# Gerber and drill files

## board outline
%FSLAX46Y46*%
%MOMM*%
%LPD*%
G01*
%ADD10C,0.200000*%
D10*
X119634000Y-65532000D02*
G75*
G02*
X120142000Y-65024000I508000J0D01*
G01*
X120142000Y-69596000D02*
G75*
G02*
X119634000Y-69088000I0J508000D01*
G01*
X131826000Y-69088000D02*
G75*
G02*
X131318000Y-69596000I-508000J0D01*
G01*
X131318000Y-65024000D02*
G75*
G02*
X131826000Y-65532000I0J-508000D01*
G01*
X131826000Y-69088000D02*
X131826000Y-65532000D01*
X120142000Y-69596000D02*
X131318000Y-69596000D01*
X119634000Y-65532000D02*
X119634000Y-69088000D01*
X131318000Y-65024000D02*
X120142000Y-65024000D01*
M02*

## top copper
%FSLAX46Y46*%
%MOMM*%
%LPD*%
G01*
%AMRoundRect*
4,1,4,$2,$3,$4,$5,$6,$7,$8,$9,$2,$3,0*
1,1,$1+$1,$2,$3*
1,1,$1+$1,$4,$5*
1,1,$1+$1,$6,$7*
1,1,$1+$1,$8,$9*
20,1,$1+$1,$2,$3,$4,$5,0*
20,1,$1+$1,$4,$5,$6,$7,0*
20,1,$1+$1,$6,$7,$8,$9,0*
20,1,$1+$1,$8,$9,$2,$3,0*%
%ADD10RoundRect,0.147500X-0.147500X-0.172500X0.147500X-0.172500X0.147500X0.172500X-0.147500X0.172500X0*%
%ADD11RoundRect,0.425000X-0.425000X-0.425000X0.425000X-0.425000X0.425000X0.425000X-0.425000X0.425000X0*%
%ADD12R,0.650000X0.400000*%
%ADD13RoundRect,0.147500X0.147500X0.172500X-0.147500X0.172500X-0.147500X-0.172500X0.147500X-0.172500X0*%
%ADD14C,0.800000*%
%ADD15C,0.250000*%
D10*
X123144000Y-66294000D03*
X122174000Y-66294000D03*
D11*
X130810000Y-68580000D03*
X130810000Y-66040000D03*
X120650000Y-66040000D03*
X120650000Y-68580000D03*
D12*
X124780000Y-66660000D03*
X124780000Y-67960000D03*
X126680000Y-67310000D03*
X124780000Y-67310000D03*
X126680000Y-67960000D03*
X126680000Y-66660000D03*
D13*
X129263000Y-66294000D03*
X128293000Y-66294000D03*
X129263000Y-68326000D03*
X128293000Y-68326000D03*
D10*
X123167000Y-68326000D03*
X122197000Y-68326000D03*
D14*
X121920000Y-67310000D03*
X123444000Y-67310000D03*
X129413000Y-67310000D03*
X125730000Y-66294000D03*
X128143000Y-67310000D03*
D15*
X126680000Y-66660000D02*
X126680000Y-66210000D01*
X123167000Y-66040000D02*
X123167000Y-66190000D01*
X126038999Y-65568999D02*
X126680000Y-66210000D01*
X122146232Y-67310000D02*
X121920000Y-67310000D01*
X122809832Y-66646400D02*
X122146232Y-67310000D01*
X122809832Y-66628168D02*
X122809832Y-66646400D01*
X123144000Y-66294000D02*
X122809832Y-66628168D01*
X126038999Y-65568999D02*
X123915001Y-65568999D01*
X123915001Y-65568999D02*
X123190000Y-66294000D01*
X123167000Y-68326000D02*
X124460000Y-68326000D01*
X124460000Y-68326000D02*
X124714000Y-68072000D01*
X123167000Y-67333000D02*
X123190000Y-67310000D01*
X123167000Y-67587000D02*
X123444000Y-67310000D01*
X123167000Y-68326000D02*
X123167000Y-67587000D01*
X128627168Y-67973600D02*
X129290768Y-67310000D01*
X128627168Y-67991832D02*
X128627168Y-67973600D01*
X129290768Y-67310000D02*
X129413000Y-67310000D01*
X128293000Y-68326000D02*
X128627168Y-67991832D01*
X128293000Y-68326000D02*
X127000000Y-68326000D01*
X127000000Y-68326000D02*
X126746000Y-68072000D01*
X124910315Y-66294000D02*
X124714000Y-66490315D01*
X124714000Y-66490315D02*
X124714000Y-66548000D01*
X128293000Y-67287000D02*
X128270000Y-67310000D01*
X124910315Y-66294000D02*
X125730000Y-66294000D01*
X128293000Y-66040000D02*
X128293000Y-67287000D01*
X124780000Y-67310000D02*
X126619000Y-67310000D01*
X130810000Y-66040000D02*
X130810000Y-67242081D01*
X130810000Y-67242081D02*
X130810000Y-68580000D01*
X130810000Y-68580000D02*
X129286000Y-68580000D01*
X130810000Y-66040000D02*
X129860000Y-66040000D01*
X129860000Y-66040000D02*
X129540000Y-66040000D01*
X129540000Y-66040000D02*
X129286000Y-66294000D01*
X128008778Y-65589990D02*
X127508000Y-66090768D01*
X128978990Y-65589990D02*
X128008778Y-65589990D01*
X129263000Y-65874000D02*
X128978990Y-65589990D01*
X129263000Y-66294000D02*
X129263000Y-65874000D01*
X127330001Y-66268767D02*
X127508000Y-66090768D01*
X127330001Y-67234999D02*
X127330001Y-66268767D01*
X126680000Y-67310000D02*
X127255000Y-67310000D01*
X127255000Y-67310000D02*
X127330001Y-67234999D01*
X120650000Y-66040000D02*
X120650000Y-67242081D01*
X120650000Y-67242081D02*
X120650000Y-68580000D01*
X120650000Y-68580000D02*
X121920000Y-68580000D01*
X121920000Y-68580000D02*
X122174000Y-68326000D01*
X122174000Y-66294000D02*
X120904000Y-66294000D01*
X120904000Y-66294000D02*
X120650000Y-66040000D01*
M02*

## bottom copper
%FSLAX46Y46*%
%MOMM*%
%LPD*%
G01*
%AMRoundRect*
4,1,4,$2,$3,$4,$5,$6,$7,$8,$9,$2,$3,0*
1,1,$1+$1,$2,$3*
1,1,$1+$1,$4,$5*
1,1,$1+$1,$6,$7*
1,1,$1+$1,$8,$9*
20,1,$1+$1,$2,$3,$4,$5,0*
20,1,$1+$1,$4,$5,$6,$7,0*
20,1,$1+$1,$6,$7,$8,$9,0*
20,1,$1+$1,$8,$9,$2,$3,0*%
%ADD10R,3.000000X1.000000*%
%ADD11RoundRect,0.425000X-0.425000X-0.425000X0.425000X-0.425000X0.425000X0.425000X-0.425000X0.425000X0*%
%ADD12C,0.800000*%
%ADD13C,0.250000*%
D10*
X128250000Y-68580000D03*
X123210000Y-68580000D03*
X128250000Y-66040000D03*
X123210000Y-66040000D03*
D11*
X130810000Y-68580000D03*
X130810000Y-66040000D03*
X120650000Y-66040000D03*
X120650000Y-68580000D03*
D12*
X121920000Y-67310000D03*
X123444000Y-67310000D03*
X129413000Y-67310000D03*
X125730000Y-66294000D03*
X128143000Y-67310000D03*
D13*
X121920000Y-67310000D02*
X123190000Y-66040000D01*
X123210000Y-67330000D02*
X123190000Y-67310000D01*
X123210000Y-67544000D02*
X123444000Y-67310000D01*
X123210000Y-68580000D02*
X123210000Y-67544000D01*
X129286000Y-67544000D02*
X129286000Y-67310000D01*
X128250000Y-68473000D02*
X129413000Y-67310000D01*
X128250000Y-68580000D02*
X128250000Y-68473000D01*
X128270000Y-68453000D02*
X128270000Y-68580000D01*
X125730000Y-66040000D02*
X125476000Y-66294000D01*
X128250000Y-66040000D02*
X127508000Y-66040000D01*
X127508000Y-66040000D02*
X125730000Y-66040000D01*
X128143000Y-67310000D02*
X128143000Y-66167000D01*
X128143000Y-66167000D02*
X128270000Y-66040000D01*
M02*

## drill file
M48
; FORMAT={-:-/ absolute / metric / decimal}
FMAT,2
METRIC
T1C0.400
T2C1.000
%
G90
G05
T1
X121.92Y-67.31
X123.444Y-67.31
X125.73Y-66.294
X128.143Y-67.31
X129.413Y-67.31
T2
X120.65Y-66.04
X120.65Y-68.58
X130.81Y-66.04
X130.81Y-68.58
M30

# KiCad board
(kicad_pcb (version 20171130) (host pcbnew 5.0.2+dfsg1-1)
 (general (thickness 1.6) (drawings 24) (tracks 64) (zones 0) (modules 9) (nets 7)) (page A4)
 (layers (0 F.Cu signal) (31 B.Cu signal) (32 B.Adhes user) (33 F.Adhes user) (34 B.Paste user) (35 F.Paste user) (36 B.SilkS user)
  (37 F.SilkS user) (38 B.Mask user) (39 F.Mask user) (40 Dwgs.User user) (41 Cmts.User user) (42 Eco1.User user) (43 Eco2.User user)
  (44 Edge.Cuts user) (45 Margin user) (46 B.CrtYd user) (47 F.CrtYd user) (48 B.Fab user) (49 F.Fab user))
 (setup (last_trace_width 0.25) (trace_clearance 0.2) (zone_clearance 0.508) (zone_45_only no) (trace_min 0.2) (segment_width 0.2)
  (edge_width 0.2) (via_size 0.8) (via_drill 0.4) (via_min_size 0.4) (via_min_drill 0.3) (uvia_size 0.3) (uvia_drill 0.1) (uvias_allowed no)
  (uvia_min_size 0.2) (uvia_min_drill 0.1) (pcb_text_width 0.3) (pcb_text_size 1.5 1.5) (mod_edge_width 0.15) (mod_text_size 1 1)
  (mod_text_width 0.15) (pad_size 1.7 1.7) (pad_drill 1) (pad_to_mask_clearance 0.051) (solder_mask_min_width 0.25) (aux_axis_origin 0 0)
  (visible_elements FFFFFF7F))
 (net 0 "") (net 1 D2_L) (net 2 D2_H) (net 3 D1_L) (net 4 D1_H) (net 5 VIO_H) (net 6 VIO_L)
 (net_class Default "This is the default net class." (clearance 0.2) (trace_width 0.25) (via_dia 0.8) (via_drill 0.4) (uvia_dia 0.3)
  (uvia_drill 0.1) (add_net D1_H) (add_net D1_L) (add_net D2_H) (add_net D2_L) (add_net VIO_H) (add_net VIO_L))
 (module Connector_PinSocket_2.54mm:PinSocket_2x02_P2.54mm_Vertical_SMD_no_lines (layer B.Cu) (at 125.73 67.31 180)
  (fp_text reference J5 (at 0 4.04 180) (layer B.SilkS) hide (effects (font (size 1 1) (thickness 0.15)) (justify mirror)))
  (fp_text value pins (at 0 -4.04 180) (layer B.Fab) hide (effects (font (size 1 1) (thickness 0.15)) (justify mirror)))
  (pad 4 smd rect (at -2.52 -1.27 180) (size 3 1) (layers B.Cu B.Paste B.Mask) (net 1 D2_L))
  (pad 3 smd rect (at 2.52 -1.27 180) (size 3 1) (layers B.Cu B.Paste B.Mask) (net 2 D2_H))
  (pad 2 smd rect (at -2.52 1.27 180) (size 3 1) (layers B.Cu B.Paste B.Mask) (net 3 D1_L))
  (pad 1 smd rect (at 2.52 1.27 180) (size 3 1) (layers B.Cu B.Paste B.Mask) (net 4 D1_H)))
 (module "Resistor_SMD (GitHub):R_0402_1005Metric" (layer F.Cu) (at 122.659 66.294)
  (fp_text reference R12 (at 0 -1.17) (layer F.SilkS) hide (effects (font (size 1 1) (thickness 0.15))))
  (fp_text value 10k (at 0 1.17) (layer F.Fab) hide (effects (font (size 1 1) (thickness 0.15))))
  (pad 2 smd roundrect (at 0.485 0) (size 0.59 0.64) (layers F.Cu F.Paste F.Mask) (roundrect_rratio 0.25) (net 4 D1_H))
  (pad 1 smd roundrect (at -0.485 0) (size 0.59 0.64) (layers F.Cu F.Paste F.Mask) (roundrect_rratio 0.25) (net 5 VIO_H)))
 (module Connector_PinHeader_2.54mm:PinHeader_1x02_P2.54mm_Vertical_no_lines (layer F.Cu) (at 130.81 66.04)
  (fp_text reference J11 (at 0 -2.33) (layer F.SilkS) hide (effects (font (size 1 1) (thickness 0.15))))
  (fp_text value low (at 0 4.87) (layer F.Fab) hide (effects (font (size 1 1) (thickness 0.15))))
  (pad 2 thru_hole roundrect (at 0 2.54) (size 1.7 1.7) (drill 1) (layers *.Cu *.Mask) (roundrect_rratio 0.25) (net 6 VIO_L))
  (pad 1 thru_hole roundrect (at 0 0) (size 1.7 1.7) (drill 1) (layers *.Cu *.Mask) (roundrect_rratio 0.25) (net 6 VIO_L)))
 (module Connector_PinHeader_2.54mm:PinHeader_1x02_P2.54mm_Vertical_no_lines (layer F.Cu) (at 120.65 66.04)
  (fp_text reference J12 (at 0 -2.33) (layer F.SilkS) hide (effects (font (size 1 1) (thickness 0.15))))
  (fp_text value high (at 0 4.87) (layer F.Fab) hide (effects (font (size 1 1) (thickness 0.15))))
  (pad 1 thru_hole roundrect (at 0 0) (size 1.7 1.7) (drill 1) (layers *.Cu *.Mask) (roundrect_rratio 0.25) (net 5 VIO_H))
  (pad 2 thru_hole roundrect (at 0 2.54) (size 1.7 1.7) (drill 1) (layers *.Cu *.Mask) (roundrect_rratio 0.25) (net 5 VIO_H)))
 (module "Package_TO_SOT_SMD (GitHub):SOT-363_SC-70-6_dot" (layer F.Cu) (at 125.73 67.31)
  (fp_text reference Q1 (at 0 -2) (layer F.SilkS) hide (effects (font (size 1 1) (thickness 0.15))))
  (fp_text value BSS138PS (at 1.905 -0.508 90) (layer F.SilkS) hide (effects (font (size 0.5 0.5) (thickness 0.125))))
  (pad 1 smd rect (at -0.95 -0.65) (size 0.65 0.4) (layers F.Cu F.Paste F.Mask) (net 3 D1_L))
  (pad 3 smd rect (at -0.95 0.65) (size 0.65 0.4) (layers F.Cu F.Paste F.Mask) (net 2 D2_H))
  (pad 5 smd rect (at 0.95 0) (size 0.65 0.4) (layers F.Cu F.Paste F.Mask) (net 6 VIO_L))
  (pad 2 smd rect (at -0.95 0) (size 0.65 0.4) (layers F.Cu F.Paste F.Mask) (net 6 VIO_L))
  (pad 4 smd rect (at 0.95 0.65) (size 0.65 0.4) (layers F.Cu F.Paste F.Mask) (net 1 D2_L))
  (pad 6 smd rect (at 0.95 -0.65) (size 0.65 0.4) (layers F.Cu F.Paste F.Mask) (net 4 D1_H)))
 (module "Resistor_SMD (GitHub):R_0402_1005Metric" (layer F.Cu) (at 128.778 66.294 180)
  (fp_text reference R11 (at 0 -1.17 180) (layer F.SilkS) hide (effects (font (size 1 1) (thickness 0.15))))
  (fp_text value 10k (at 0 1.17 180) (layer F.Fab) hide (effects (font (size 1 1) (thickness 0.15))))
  (pad 1 smd roundrect (at -0.485 0 180) (size 0.59 0.64) (layers F.Cu F.Paste F.Mask) (roundrect_rratio 0.25) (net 6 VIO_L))
  (pad 2 smd roundrect (at 0.485 0 180) (size 0.59 0.64) (layers F.Cu F.Paste F.Mask) (roundrect_rratio 0.25) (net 3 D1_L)))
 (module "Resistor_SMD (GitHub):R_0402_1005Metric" (layer F.Cu) (at 128.778 68.326 180)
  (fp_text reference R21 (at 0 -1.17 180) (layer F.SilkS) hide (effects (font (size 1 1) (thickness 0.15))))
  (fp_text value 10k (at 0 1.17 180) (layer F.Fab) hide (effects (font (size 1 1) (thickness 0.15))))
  (pad 1 smd roundrect (at -0.485 0 180) (size 0.59 0.64) (layers F.Cu F.Paste F.Mask) (roundrect_rratio 0.25) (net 6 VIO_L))
  (pad 2 smd roundrect (at 0.485 0 180) (size 0.59 0.64) (layers F.Cu F.Paste F.Mask) (roundrect_rratio 0.25) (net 1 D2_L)))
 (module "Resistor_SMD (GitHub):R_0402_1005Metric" (layer F.Cu) (at 122.682 68.326)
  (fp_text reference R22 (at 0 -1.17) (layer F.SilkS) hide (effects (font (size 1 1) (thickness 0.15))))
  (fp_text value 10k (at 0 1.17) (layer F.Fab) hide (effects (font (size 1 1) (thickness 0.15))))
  (pad 2 smd roundrect (at 0.485 0) (size 0.59 0.64) (layers F.Cu F.Paste F.Mask) (roundrect_rratio 0.25) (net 2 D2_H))
  (pad 1 smd roundrect (at -0.485 0) (size 0.59 0.64) (layers F.Cu F.Paste F.Mask) (roundrect_rratio 0.25) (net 5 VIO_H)))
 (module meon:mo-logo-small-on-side (layer B.Cu) (at 125.73 67.31 180)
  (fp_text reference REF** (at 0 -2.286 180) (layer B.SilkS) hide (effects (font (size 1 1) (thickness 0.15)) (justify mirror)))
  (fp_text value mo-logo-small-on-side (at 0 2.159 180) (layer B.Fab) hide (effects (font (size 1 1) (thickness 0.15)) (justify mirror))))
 (gr_arc (start 120.142 65.532) (end 120.142 65.024) (angle -90) (layer Edge.Cuts) (width 0.2))
 (gr_arc (start 120.142 69.088) (end 119.634 69.088) (angle -90) (layer Edge.Cuts) (width 0.2))
 (gr_arc (start 131.318 69.088) (end 131.318 69.596) (angle -90) (layer Edge.Cuts) (width 0.2))
 (gr_arc (start 131.318 65.532) (end 131.826 65.532) (angle -90) (layer Edge.Cuts) (width 0.2))
 (gr_line (start 131.826 69.088) (end 131.826 65.532) (layer Edge.Cuts) (width 0.2))
 (gr_line (start 120.142 69.596) (end 131.318 69.596) (layer Edge.Cuts) (width 0.2))
 (gr_line (start 119.634 65.532) (end 119.634 69.088) (layer Edge.Cuts) (width 0.2))
 (gr_line (start 131.318 65.024) (end 120.142 65.024) (layer Edge.Cuts) (width 0.2))
 (via (at 121.92 67.31) (size 0.8) (drill 0.4) (layers F.Cu B.Cu) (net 4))
 (segment (start 126.68 66.66) (end 126.68 66.21) (width 0.25) (layer F.Cu) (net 4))
 (segment (start 123.167 66.04) (end 123.167 66.19) (width 0.25) (layer F.Cu) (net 4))
 (segment (start 126.038999 65.568999) (end 126.68 66.21) (width 0.25) (layer F.Cu) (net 4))
 (segment (start 122.146232 67.31) (end 121.92 67.31) (width 0.25) (layer F.Cu) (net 4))
 (segment (start 122.809832 66.6464) (end 122.146232 67.31) (width 0.25) (layer F.Cu) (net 4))
 (segment (start 122.809832 66.628168) (end 122.809832 66.6464) (width 0.25) (layer F.Cu) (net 4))
 (segment (start 123.144 66.294) (end 122.809832 66.628168) (width 0.25) (layer F.Cu) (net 4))
 (segment (start 126.038999 65.568999) (end 123.915001 65.568999) (width 0.25) (layer F.Cu) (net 4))
 (segment (start 123.915001 65.568999) (end 123.19 66.294) (width 0.25) (layer F.Cu) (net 4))
 (segment (start 121.92 67.31) (end 123.19 66.04) (width 0.25) (layer B.Cu) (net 4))
 (via (at 123.444 67.31) (size 0.8) (drill 0.4) (layers F.Cu B.Cu) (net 2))
 (segment (start 123.21 67.33) (end 123.19 67.31) (width 0.25) (layer B.Cu) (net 2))
 (segment (start 123.167 68.326) (end 124.46 68.326) (width 0.25) (layer F.Cu) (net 2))
 (segment (start 124.46 68.326) (end 124.714 68.072) (width 0.25) (layer F.Cu) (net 2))
 (segment (start 123.167 67.333) (end 123.19 67.31) (width 0.25) (layer F.Cu) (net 2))
 (segment (start 123.167 67.587) (end 123.444 67.31) (width 0.25) (layer F.Cu) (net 2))
 (segment (start 123.167 68.326) (end 123.167 67.587) (width 0.25) (layer F.Cu) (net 2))
 (segment (start 123.21 67.544) (end 123.444 67.31) (width 0.25) (layer B.Cu) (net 2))
 (segment (start 123.21 68.58) (end 123.21 67.544) (width 0.25) (layer B.Cu) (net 2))
 (via (at 129.413 67.31) (size 0.8) (drill 0.4) (layers F.Cu B.Cu) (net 1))
 (segment (start 129.286 67.544) (end 129.286 67.31) (width 0.25) (layer B.Cu) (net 1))
 (segment (start 128.25 68.473) (end 129.413 67.31) (width 0.25) (layer B.Cu) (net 1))
 (segment (start 128.25 68.58) (end 128.25 68.473) (width 0.25) (layer B.Cu) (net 1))
 (segment (start 128.27 68.453) (end 128.27 68.58) (width 0.25) (layer B.Cu) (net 1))
 (segment (start 128.627168 67.9736) (end 129.290768 67.31) (width 0.25) (layer F.Cu) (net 1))
 (segment (start 128.627168 67.991832) (end 128.627168 67.9736) (width 0.25) (layer F.Cu) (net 1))
 (segment (start 129.290768 67.31) (end 129.413 67.31) (width 0.25) (layer F.Cu) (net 1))
 (segment (start 128.293 68.326) (end 128.627168 67.991832) (width 0.25) (layer F.Cu) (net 1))
 (segment (start 128.293 68.326) (end 127 68.326) (width 0.25) (layer F.Cu) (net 1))
 (segment (start 127 68.326) (end 126.746 68.072) (width 0.25) (layer F.Cu) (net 1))
 (via (at 125.73 66.294) (size 0.8) (drill 0.4) (layers F.Cu B.Cu) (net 3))
 (segment (start 124.910315 66.294) (end 124.714 66.490315) (width 0.25) (layer F.Cu) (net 3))
 (segment (start 124.714 66.490315) (end 124.714 66.548) (width 0.25) (layer F.Cu) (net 3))
 (segment (start 125.73 66.04) (end 125.476 66.294) (width 0.25) (layer B.Cu) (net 3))
 (segment (start 128.25 66.04) (end 127.508 66.04) (width 0.25) (layer B.Cu) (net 3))
 (segment (start 127.508 66.04) (end 125.73 66.04) (width 0.25) (layer B.Cu) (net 3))
 (via (at 128.143 67.31) (size 0.8) (drill 0.4) (layers F.Cu B.Cu) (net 3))
 (segment (start 128.293 67.287) (end 128.27 67.31) (width 0.25) (layer F.Cu) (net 3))
 (segment (start 124.910315 66.294) (end 125.73 66.294) (width 0.25) (layer F.Cu) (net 3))
 (segment (start 128.293 66.04) (end 128.293 67.287) (width 0.25) (layer F.Cu) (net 3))
 (segment (start 128.143 67.31) (end 128.143 66.167) (width 0.25) (layer B.Cu) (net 3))
 (segment (start 128.143 66.167) (end 128.27 66.04) (width 0.25) (layer B.Cu) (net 3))
 (segment (start 124.78 67.31) (end 126.619 67.31) (width 0.25) (layer F.Cu) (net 6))
 (segment (start 130.81 66.04) (end 130.81 67.242081) (width 0.25) (layer F.Cu) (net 6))
 (segment (start 130.81 67.242081) (end 130.81 68.58) (width 0.25) (layer F.Cu) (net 6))
 (segment (start 130.81 68.58) (end 129.286 68.58) (width 0.25) (layer F.Cu) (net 6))
 (segment (start 130.81 66.04) (end 129.86 66.04) (width 0.25) (layer F.Cu) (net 6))
 (segment (start 129.86 66.04) (end 129.54 66.04) (width 0.25) (layer F.Cu) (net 6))
 (segment (start 129.54 66.04) (end 129.286 66.294) (width 0.25) (layer F.Cu) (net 6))
 (segment (start 128.008778 65.58999) (end 127.508 66.090768) (width 0.25) (layer F.Cu) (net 6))
 (segment (start 128.97899 65.58999) (end 128.008778 65.58999) (width 0.25) (layer F.Cu) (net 6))
 (segment (start 129.263 65.874) (end 128.97899 65.58999) (width 0.25) (layer F.Cu) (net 6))
 (segment (start 129.263 66.294) (end 129.263 65.874) (width 0.25) (layer F.Cu) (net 6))
 (segment (start 127.330001 66.268767) (end 127.508 66.090768) (width 0.25) (layer F.Cu) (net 6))
 (segment (start 127.330001 67.234999) (end 127.330001 66.268767) (width 0.25) (layer F.Cu) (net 6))
 (segment (start 126.68 67.31) (end 127.255 67.31) (width 0.25) (layer F.Cu) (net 6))
 (segment (start 127.255 67.31) (end 127.330001 67.234999) (width 0.25) (layer F.Cu) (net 6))
 (segment (start 120.65 66.04) (end 120.65 67.242081) (width 0.25) (layer F.Cu) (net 5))
 (segment (start 120.65 67.242081) (end 120.65 68.58) (width 0.25) (layer F.Cu) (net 5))
 (segment (start 120.65 68.58) (end 121.92 68.58) (width 0.25) (layer F.Cu) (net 5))
 (segment (start 121.92 68.58) (end 122.174 68.326) (width 0.25) (layer F.Cu) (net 5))
 (segment (start 122.174 66.294) (end 120.904 66.294) (width 0.25) (layer F.Cu) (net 5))
 (segment (start 120.904 66.294) (end 120.65 66.04) (width 0.25) (layer F.Cu) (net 5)))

